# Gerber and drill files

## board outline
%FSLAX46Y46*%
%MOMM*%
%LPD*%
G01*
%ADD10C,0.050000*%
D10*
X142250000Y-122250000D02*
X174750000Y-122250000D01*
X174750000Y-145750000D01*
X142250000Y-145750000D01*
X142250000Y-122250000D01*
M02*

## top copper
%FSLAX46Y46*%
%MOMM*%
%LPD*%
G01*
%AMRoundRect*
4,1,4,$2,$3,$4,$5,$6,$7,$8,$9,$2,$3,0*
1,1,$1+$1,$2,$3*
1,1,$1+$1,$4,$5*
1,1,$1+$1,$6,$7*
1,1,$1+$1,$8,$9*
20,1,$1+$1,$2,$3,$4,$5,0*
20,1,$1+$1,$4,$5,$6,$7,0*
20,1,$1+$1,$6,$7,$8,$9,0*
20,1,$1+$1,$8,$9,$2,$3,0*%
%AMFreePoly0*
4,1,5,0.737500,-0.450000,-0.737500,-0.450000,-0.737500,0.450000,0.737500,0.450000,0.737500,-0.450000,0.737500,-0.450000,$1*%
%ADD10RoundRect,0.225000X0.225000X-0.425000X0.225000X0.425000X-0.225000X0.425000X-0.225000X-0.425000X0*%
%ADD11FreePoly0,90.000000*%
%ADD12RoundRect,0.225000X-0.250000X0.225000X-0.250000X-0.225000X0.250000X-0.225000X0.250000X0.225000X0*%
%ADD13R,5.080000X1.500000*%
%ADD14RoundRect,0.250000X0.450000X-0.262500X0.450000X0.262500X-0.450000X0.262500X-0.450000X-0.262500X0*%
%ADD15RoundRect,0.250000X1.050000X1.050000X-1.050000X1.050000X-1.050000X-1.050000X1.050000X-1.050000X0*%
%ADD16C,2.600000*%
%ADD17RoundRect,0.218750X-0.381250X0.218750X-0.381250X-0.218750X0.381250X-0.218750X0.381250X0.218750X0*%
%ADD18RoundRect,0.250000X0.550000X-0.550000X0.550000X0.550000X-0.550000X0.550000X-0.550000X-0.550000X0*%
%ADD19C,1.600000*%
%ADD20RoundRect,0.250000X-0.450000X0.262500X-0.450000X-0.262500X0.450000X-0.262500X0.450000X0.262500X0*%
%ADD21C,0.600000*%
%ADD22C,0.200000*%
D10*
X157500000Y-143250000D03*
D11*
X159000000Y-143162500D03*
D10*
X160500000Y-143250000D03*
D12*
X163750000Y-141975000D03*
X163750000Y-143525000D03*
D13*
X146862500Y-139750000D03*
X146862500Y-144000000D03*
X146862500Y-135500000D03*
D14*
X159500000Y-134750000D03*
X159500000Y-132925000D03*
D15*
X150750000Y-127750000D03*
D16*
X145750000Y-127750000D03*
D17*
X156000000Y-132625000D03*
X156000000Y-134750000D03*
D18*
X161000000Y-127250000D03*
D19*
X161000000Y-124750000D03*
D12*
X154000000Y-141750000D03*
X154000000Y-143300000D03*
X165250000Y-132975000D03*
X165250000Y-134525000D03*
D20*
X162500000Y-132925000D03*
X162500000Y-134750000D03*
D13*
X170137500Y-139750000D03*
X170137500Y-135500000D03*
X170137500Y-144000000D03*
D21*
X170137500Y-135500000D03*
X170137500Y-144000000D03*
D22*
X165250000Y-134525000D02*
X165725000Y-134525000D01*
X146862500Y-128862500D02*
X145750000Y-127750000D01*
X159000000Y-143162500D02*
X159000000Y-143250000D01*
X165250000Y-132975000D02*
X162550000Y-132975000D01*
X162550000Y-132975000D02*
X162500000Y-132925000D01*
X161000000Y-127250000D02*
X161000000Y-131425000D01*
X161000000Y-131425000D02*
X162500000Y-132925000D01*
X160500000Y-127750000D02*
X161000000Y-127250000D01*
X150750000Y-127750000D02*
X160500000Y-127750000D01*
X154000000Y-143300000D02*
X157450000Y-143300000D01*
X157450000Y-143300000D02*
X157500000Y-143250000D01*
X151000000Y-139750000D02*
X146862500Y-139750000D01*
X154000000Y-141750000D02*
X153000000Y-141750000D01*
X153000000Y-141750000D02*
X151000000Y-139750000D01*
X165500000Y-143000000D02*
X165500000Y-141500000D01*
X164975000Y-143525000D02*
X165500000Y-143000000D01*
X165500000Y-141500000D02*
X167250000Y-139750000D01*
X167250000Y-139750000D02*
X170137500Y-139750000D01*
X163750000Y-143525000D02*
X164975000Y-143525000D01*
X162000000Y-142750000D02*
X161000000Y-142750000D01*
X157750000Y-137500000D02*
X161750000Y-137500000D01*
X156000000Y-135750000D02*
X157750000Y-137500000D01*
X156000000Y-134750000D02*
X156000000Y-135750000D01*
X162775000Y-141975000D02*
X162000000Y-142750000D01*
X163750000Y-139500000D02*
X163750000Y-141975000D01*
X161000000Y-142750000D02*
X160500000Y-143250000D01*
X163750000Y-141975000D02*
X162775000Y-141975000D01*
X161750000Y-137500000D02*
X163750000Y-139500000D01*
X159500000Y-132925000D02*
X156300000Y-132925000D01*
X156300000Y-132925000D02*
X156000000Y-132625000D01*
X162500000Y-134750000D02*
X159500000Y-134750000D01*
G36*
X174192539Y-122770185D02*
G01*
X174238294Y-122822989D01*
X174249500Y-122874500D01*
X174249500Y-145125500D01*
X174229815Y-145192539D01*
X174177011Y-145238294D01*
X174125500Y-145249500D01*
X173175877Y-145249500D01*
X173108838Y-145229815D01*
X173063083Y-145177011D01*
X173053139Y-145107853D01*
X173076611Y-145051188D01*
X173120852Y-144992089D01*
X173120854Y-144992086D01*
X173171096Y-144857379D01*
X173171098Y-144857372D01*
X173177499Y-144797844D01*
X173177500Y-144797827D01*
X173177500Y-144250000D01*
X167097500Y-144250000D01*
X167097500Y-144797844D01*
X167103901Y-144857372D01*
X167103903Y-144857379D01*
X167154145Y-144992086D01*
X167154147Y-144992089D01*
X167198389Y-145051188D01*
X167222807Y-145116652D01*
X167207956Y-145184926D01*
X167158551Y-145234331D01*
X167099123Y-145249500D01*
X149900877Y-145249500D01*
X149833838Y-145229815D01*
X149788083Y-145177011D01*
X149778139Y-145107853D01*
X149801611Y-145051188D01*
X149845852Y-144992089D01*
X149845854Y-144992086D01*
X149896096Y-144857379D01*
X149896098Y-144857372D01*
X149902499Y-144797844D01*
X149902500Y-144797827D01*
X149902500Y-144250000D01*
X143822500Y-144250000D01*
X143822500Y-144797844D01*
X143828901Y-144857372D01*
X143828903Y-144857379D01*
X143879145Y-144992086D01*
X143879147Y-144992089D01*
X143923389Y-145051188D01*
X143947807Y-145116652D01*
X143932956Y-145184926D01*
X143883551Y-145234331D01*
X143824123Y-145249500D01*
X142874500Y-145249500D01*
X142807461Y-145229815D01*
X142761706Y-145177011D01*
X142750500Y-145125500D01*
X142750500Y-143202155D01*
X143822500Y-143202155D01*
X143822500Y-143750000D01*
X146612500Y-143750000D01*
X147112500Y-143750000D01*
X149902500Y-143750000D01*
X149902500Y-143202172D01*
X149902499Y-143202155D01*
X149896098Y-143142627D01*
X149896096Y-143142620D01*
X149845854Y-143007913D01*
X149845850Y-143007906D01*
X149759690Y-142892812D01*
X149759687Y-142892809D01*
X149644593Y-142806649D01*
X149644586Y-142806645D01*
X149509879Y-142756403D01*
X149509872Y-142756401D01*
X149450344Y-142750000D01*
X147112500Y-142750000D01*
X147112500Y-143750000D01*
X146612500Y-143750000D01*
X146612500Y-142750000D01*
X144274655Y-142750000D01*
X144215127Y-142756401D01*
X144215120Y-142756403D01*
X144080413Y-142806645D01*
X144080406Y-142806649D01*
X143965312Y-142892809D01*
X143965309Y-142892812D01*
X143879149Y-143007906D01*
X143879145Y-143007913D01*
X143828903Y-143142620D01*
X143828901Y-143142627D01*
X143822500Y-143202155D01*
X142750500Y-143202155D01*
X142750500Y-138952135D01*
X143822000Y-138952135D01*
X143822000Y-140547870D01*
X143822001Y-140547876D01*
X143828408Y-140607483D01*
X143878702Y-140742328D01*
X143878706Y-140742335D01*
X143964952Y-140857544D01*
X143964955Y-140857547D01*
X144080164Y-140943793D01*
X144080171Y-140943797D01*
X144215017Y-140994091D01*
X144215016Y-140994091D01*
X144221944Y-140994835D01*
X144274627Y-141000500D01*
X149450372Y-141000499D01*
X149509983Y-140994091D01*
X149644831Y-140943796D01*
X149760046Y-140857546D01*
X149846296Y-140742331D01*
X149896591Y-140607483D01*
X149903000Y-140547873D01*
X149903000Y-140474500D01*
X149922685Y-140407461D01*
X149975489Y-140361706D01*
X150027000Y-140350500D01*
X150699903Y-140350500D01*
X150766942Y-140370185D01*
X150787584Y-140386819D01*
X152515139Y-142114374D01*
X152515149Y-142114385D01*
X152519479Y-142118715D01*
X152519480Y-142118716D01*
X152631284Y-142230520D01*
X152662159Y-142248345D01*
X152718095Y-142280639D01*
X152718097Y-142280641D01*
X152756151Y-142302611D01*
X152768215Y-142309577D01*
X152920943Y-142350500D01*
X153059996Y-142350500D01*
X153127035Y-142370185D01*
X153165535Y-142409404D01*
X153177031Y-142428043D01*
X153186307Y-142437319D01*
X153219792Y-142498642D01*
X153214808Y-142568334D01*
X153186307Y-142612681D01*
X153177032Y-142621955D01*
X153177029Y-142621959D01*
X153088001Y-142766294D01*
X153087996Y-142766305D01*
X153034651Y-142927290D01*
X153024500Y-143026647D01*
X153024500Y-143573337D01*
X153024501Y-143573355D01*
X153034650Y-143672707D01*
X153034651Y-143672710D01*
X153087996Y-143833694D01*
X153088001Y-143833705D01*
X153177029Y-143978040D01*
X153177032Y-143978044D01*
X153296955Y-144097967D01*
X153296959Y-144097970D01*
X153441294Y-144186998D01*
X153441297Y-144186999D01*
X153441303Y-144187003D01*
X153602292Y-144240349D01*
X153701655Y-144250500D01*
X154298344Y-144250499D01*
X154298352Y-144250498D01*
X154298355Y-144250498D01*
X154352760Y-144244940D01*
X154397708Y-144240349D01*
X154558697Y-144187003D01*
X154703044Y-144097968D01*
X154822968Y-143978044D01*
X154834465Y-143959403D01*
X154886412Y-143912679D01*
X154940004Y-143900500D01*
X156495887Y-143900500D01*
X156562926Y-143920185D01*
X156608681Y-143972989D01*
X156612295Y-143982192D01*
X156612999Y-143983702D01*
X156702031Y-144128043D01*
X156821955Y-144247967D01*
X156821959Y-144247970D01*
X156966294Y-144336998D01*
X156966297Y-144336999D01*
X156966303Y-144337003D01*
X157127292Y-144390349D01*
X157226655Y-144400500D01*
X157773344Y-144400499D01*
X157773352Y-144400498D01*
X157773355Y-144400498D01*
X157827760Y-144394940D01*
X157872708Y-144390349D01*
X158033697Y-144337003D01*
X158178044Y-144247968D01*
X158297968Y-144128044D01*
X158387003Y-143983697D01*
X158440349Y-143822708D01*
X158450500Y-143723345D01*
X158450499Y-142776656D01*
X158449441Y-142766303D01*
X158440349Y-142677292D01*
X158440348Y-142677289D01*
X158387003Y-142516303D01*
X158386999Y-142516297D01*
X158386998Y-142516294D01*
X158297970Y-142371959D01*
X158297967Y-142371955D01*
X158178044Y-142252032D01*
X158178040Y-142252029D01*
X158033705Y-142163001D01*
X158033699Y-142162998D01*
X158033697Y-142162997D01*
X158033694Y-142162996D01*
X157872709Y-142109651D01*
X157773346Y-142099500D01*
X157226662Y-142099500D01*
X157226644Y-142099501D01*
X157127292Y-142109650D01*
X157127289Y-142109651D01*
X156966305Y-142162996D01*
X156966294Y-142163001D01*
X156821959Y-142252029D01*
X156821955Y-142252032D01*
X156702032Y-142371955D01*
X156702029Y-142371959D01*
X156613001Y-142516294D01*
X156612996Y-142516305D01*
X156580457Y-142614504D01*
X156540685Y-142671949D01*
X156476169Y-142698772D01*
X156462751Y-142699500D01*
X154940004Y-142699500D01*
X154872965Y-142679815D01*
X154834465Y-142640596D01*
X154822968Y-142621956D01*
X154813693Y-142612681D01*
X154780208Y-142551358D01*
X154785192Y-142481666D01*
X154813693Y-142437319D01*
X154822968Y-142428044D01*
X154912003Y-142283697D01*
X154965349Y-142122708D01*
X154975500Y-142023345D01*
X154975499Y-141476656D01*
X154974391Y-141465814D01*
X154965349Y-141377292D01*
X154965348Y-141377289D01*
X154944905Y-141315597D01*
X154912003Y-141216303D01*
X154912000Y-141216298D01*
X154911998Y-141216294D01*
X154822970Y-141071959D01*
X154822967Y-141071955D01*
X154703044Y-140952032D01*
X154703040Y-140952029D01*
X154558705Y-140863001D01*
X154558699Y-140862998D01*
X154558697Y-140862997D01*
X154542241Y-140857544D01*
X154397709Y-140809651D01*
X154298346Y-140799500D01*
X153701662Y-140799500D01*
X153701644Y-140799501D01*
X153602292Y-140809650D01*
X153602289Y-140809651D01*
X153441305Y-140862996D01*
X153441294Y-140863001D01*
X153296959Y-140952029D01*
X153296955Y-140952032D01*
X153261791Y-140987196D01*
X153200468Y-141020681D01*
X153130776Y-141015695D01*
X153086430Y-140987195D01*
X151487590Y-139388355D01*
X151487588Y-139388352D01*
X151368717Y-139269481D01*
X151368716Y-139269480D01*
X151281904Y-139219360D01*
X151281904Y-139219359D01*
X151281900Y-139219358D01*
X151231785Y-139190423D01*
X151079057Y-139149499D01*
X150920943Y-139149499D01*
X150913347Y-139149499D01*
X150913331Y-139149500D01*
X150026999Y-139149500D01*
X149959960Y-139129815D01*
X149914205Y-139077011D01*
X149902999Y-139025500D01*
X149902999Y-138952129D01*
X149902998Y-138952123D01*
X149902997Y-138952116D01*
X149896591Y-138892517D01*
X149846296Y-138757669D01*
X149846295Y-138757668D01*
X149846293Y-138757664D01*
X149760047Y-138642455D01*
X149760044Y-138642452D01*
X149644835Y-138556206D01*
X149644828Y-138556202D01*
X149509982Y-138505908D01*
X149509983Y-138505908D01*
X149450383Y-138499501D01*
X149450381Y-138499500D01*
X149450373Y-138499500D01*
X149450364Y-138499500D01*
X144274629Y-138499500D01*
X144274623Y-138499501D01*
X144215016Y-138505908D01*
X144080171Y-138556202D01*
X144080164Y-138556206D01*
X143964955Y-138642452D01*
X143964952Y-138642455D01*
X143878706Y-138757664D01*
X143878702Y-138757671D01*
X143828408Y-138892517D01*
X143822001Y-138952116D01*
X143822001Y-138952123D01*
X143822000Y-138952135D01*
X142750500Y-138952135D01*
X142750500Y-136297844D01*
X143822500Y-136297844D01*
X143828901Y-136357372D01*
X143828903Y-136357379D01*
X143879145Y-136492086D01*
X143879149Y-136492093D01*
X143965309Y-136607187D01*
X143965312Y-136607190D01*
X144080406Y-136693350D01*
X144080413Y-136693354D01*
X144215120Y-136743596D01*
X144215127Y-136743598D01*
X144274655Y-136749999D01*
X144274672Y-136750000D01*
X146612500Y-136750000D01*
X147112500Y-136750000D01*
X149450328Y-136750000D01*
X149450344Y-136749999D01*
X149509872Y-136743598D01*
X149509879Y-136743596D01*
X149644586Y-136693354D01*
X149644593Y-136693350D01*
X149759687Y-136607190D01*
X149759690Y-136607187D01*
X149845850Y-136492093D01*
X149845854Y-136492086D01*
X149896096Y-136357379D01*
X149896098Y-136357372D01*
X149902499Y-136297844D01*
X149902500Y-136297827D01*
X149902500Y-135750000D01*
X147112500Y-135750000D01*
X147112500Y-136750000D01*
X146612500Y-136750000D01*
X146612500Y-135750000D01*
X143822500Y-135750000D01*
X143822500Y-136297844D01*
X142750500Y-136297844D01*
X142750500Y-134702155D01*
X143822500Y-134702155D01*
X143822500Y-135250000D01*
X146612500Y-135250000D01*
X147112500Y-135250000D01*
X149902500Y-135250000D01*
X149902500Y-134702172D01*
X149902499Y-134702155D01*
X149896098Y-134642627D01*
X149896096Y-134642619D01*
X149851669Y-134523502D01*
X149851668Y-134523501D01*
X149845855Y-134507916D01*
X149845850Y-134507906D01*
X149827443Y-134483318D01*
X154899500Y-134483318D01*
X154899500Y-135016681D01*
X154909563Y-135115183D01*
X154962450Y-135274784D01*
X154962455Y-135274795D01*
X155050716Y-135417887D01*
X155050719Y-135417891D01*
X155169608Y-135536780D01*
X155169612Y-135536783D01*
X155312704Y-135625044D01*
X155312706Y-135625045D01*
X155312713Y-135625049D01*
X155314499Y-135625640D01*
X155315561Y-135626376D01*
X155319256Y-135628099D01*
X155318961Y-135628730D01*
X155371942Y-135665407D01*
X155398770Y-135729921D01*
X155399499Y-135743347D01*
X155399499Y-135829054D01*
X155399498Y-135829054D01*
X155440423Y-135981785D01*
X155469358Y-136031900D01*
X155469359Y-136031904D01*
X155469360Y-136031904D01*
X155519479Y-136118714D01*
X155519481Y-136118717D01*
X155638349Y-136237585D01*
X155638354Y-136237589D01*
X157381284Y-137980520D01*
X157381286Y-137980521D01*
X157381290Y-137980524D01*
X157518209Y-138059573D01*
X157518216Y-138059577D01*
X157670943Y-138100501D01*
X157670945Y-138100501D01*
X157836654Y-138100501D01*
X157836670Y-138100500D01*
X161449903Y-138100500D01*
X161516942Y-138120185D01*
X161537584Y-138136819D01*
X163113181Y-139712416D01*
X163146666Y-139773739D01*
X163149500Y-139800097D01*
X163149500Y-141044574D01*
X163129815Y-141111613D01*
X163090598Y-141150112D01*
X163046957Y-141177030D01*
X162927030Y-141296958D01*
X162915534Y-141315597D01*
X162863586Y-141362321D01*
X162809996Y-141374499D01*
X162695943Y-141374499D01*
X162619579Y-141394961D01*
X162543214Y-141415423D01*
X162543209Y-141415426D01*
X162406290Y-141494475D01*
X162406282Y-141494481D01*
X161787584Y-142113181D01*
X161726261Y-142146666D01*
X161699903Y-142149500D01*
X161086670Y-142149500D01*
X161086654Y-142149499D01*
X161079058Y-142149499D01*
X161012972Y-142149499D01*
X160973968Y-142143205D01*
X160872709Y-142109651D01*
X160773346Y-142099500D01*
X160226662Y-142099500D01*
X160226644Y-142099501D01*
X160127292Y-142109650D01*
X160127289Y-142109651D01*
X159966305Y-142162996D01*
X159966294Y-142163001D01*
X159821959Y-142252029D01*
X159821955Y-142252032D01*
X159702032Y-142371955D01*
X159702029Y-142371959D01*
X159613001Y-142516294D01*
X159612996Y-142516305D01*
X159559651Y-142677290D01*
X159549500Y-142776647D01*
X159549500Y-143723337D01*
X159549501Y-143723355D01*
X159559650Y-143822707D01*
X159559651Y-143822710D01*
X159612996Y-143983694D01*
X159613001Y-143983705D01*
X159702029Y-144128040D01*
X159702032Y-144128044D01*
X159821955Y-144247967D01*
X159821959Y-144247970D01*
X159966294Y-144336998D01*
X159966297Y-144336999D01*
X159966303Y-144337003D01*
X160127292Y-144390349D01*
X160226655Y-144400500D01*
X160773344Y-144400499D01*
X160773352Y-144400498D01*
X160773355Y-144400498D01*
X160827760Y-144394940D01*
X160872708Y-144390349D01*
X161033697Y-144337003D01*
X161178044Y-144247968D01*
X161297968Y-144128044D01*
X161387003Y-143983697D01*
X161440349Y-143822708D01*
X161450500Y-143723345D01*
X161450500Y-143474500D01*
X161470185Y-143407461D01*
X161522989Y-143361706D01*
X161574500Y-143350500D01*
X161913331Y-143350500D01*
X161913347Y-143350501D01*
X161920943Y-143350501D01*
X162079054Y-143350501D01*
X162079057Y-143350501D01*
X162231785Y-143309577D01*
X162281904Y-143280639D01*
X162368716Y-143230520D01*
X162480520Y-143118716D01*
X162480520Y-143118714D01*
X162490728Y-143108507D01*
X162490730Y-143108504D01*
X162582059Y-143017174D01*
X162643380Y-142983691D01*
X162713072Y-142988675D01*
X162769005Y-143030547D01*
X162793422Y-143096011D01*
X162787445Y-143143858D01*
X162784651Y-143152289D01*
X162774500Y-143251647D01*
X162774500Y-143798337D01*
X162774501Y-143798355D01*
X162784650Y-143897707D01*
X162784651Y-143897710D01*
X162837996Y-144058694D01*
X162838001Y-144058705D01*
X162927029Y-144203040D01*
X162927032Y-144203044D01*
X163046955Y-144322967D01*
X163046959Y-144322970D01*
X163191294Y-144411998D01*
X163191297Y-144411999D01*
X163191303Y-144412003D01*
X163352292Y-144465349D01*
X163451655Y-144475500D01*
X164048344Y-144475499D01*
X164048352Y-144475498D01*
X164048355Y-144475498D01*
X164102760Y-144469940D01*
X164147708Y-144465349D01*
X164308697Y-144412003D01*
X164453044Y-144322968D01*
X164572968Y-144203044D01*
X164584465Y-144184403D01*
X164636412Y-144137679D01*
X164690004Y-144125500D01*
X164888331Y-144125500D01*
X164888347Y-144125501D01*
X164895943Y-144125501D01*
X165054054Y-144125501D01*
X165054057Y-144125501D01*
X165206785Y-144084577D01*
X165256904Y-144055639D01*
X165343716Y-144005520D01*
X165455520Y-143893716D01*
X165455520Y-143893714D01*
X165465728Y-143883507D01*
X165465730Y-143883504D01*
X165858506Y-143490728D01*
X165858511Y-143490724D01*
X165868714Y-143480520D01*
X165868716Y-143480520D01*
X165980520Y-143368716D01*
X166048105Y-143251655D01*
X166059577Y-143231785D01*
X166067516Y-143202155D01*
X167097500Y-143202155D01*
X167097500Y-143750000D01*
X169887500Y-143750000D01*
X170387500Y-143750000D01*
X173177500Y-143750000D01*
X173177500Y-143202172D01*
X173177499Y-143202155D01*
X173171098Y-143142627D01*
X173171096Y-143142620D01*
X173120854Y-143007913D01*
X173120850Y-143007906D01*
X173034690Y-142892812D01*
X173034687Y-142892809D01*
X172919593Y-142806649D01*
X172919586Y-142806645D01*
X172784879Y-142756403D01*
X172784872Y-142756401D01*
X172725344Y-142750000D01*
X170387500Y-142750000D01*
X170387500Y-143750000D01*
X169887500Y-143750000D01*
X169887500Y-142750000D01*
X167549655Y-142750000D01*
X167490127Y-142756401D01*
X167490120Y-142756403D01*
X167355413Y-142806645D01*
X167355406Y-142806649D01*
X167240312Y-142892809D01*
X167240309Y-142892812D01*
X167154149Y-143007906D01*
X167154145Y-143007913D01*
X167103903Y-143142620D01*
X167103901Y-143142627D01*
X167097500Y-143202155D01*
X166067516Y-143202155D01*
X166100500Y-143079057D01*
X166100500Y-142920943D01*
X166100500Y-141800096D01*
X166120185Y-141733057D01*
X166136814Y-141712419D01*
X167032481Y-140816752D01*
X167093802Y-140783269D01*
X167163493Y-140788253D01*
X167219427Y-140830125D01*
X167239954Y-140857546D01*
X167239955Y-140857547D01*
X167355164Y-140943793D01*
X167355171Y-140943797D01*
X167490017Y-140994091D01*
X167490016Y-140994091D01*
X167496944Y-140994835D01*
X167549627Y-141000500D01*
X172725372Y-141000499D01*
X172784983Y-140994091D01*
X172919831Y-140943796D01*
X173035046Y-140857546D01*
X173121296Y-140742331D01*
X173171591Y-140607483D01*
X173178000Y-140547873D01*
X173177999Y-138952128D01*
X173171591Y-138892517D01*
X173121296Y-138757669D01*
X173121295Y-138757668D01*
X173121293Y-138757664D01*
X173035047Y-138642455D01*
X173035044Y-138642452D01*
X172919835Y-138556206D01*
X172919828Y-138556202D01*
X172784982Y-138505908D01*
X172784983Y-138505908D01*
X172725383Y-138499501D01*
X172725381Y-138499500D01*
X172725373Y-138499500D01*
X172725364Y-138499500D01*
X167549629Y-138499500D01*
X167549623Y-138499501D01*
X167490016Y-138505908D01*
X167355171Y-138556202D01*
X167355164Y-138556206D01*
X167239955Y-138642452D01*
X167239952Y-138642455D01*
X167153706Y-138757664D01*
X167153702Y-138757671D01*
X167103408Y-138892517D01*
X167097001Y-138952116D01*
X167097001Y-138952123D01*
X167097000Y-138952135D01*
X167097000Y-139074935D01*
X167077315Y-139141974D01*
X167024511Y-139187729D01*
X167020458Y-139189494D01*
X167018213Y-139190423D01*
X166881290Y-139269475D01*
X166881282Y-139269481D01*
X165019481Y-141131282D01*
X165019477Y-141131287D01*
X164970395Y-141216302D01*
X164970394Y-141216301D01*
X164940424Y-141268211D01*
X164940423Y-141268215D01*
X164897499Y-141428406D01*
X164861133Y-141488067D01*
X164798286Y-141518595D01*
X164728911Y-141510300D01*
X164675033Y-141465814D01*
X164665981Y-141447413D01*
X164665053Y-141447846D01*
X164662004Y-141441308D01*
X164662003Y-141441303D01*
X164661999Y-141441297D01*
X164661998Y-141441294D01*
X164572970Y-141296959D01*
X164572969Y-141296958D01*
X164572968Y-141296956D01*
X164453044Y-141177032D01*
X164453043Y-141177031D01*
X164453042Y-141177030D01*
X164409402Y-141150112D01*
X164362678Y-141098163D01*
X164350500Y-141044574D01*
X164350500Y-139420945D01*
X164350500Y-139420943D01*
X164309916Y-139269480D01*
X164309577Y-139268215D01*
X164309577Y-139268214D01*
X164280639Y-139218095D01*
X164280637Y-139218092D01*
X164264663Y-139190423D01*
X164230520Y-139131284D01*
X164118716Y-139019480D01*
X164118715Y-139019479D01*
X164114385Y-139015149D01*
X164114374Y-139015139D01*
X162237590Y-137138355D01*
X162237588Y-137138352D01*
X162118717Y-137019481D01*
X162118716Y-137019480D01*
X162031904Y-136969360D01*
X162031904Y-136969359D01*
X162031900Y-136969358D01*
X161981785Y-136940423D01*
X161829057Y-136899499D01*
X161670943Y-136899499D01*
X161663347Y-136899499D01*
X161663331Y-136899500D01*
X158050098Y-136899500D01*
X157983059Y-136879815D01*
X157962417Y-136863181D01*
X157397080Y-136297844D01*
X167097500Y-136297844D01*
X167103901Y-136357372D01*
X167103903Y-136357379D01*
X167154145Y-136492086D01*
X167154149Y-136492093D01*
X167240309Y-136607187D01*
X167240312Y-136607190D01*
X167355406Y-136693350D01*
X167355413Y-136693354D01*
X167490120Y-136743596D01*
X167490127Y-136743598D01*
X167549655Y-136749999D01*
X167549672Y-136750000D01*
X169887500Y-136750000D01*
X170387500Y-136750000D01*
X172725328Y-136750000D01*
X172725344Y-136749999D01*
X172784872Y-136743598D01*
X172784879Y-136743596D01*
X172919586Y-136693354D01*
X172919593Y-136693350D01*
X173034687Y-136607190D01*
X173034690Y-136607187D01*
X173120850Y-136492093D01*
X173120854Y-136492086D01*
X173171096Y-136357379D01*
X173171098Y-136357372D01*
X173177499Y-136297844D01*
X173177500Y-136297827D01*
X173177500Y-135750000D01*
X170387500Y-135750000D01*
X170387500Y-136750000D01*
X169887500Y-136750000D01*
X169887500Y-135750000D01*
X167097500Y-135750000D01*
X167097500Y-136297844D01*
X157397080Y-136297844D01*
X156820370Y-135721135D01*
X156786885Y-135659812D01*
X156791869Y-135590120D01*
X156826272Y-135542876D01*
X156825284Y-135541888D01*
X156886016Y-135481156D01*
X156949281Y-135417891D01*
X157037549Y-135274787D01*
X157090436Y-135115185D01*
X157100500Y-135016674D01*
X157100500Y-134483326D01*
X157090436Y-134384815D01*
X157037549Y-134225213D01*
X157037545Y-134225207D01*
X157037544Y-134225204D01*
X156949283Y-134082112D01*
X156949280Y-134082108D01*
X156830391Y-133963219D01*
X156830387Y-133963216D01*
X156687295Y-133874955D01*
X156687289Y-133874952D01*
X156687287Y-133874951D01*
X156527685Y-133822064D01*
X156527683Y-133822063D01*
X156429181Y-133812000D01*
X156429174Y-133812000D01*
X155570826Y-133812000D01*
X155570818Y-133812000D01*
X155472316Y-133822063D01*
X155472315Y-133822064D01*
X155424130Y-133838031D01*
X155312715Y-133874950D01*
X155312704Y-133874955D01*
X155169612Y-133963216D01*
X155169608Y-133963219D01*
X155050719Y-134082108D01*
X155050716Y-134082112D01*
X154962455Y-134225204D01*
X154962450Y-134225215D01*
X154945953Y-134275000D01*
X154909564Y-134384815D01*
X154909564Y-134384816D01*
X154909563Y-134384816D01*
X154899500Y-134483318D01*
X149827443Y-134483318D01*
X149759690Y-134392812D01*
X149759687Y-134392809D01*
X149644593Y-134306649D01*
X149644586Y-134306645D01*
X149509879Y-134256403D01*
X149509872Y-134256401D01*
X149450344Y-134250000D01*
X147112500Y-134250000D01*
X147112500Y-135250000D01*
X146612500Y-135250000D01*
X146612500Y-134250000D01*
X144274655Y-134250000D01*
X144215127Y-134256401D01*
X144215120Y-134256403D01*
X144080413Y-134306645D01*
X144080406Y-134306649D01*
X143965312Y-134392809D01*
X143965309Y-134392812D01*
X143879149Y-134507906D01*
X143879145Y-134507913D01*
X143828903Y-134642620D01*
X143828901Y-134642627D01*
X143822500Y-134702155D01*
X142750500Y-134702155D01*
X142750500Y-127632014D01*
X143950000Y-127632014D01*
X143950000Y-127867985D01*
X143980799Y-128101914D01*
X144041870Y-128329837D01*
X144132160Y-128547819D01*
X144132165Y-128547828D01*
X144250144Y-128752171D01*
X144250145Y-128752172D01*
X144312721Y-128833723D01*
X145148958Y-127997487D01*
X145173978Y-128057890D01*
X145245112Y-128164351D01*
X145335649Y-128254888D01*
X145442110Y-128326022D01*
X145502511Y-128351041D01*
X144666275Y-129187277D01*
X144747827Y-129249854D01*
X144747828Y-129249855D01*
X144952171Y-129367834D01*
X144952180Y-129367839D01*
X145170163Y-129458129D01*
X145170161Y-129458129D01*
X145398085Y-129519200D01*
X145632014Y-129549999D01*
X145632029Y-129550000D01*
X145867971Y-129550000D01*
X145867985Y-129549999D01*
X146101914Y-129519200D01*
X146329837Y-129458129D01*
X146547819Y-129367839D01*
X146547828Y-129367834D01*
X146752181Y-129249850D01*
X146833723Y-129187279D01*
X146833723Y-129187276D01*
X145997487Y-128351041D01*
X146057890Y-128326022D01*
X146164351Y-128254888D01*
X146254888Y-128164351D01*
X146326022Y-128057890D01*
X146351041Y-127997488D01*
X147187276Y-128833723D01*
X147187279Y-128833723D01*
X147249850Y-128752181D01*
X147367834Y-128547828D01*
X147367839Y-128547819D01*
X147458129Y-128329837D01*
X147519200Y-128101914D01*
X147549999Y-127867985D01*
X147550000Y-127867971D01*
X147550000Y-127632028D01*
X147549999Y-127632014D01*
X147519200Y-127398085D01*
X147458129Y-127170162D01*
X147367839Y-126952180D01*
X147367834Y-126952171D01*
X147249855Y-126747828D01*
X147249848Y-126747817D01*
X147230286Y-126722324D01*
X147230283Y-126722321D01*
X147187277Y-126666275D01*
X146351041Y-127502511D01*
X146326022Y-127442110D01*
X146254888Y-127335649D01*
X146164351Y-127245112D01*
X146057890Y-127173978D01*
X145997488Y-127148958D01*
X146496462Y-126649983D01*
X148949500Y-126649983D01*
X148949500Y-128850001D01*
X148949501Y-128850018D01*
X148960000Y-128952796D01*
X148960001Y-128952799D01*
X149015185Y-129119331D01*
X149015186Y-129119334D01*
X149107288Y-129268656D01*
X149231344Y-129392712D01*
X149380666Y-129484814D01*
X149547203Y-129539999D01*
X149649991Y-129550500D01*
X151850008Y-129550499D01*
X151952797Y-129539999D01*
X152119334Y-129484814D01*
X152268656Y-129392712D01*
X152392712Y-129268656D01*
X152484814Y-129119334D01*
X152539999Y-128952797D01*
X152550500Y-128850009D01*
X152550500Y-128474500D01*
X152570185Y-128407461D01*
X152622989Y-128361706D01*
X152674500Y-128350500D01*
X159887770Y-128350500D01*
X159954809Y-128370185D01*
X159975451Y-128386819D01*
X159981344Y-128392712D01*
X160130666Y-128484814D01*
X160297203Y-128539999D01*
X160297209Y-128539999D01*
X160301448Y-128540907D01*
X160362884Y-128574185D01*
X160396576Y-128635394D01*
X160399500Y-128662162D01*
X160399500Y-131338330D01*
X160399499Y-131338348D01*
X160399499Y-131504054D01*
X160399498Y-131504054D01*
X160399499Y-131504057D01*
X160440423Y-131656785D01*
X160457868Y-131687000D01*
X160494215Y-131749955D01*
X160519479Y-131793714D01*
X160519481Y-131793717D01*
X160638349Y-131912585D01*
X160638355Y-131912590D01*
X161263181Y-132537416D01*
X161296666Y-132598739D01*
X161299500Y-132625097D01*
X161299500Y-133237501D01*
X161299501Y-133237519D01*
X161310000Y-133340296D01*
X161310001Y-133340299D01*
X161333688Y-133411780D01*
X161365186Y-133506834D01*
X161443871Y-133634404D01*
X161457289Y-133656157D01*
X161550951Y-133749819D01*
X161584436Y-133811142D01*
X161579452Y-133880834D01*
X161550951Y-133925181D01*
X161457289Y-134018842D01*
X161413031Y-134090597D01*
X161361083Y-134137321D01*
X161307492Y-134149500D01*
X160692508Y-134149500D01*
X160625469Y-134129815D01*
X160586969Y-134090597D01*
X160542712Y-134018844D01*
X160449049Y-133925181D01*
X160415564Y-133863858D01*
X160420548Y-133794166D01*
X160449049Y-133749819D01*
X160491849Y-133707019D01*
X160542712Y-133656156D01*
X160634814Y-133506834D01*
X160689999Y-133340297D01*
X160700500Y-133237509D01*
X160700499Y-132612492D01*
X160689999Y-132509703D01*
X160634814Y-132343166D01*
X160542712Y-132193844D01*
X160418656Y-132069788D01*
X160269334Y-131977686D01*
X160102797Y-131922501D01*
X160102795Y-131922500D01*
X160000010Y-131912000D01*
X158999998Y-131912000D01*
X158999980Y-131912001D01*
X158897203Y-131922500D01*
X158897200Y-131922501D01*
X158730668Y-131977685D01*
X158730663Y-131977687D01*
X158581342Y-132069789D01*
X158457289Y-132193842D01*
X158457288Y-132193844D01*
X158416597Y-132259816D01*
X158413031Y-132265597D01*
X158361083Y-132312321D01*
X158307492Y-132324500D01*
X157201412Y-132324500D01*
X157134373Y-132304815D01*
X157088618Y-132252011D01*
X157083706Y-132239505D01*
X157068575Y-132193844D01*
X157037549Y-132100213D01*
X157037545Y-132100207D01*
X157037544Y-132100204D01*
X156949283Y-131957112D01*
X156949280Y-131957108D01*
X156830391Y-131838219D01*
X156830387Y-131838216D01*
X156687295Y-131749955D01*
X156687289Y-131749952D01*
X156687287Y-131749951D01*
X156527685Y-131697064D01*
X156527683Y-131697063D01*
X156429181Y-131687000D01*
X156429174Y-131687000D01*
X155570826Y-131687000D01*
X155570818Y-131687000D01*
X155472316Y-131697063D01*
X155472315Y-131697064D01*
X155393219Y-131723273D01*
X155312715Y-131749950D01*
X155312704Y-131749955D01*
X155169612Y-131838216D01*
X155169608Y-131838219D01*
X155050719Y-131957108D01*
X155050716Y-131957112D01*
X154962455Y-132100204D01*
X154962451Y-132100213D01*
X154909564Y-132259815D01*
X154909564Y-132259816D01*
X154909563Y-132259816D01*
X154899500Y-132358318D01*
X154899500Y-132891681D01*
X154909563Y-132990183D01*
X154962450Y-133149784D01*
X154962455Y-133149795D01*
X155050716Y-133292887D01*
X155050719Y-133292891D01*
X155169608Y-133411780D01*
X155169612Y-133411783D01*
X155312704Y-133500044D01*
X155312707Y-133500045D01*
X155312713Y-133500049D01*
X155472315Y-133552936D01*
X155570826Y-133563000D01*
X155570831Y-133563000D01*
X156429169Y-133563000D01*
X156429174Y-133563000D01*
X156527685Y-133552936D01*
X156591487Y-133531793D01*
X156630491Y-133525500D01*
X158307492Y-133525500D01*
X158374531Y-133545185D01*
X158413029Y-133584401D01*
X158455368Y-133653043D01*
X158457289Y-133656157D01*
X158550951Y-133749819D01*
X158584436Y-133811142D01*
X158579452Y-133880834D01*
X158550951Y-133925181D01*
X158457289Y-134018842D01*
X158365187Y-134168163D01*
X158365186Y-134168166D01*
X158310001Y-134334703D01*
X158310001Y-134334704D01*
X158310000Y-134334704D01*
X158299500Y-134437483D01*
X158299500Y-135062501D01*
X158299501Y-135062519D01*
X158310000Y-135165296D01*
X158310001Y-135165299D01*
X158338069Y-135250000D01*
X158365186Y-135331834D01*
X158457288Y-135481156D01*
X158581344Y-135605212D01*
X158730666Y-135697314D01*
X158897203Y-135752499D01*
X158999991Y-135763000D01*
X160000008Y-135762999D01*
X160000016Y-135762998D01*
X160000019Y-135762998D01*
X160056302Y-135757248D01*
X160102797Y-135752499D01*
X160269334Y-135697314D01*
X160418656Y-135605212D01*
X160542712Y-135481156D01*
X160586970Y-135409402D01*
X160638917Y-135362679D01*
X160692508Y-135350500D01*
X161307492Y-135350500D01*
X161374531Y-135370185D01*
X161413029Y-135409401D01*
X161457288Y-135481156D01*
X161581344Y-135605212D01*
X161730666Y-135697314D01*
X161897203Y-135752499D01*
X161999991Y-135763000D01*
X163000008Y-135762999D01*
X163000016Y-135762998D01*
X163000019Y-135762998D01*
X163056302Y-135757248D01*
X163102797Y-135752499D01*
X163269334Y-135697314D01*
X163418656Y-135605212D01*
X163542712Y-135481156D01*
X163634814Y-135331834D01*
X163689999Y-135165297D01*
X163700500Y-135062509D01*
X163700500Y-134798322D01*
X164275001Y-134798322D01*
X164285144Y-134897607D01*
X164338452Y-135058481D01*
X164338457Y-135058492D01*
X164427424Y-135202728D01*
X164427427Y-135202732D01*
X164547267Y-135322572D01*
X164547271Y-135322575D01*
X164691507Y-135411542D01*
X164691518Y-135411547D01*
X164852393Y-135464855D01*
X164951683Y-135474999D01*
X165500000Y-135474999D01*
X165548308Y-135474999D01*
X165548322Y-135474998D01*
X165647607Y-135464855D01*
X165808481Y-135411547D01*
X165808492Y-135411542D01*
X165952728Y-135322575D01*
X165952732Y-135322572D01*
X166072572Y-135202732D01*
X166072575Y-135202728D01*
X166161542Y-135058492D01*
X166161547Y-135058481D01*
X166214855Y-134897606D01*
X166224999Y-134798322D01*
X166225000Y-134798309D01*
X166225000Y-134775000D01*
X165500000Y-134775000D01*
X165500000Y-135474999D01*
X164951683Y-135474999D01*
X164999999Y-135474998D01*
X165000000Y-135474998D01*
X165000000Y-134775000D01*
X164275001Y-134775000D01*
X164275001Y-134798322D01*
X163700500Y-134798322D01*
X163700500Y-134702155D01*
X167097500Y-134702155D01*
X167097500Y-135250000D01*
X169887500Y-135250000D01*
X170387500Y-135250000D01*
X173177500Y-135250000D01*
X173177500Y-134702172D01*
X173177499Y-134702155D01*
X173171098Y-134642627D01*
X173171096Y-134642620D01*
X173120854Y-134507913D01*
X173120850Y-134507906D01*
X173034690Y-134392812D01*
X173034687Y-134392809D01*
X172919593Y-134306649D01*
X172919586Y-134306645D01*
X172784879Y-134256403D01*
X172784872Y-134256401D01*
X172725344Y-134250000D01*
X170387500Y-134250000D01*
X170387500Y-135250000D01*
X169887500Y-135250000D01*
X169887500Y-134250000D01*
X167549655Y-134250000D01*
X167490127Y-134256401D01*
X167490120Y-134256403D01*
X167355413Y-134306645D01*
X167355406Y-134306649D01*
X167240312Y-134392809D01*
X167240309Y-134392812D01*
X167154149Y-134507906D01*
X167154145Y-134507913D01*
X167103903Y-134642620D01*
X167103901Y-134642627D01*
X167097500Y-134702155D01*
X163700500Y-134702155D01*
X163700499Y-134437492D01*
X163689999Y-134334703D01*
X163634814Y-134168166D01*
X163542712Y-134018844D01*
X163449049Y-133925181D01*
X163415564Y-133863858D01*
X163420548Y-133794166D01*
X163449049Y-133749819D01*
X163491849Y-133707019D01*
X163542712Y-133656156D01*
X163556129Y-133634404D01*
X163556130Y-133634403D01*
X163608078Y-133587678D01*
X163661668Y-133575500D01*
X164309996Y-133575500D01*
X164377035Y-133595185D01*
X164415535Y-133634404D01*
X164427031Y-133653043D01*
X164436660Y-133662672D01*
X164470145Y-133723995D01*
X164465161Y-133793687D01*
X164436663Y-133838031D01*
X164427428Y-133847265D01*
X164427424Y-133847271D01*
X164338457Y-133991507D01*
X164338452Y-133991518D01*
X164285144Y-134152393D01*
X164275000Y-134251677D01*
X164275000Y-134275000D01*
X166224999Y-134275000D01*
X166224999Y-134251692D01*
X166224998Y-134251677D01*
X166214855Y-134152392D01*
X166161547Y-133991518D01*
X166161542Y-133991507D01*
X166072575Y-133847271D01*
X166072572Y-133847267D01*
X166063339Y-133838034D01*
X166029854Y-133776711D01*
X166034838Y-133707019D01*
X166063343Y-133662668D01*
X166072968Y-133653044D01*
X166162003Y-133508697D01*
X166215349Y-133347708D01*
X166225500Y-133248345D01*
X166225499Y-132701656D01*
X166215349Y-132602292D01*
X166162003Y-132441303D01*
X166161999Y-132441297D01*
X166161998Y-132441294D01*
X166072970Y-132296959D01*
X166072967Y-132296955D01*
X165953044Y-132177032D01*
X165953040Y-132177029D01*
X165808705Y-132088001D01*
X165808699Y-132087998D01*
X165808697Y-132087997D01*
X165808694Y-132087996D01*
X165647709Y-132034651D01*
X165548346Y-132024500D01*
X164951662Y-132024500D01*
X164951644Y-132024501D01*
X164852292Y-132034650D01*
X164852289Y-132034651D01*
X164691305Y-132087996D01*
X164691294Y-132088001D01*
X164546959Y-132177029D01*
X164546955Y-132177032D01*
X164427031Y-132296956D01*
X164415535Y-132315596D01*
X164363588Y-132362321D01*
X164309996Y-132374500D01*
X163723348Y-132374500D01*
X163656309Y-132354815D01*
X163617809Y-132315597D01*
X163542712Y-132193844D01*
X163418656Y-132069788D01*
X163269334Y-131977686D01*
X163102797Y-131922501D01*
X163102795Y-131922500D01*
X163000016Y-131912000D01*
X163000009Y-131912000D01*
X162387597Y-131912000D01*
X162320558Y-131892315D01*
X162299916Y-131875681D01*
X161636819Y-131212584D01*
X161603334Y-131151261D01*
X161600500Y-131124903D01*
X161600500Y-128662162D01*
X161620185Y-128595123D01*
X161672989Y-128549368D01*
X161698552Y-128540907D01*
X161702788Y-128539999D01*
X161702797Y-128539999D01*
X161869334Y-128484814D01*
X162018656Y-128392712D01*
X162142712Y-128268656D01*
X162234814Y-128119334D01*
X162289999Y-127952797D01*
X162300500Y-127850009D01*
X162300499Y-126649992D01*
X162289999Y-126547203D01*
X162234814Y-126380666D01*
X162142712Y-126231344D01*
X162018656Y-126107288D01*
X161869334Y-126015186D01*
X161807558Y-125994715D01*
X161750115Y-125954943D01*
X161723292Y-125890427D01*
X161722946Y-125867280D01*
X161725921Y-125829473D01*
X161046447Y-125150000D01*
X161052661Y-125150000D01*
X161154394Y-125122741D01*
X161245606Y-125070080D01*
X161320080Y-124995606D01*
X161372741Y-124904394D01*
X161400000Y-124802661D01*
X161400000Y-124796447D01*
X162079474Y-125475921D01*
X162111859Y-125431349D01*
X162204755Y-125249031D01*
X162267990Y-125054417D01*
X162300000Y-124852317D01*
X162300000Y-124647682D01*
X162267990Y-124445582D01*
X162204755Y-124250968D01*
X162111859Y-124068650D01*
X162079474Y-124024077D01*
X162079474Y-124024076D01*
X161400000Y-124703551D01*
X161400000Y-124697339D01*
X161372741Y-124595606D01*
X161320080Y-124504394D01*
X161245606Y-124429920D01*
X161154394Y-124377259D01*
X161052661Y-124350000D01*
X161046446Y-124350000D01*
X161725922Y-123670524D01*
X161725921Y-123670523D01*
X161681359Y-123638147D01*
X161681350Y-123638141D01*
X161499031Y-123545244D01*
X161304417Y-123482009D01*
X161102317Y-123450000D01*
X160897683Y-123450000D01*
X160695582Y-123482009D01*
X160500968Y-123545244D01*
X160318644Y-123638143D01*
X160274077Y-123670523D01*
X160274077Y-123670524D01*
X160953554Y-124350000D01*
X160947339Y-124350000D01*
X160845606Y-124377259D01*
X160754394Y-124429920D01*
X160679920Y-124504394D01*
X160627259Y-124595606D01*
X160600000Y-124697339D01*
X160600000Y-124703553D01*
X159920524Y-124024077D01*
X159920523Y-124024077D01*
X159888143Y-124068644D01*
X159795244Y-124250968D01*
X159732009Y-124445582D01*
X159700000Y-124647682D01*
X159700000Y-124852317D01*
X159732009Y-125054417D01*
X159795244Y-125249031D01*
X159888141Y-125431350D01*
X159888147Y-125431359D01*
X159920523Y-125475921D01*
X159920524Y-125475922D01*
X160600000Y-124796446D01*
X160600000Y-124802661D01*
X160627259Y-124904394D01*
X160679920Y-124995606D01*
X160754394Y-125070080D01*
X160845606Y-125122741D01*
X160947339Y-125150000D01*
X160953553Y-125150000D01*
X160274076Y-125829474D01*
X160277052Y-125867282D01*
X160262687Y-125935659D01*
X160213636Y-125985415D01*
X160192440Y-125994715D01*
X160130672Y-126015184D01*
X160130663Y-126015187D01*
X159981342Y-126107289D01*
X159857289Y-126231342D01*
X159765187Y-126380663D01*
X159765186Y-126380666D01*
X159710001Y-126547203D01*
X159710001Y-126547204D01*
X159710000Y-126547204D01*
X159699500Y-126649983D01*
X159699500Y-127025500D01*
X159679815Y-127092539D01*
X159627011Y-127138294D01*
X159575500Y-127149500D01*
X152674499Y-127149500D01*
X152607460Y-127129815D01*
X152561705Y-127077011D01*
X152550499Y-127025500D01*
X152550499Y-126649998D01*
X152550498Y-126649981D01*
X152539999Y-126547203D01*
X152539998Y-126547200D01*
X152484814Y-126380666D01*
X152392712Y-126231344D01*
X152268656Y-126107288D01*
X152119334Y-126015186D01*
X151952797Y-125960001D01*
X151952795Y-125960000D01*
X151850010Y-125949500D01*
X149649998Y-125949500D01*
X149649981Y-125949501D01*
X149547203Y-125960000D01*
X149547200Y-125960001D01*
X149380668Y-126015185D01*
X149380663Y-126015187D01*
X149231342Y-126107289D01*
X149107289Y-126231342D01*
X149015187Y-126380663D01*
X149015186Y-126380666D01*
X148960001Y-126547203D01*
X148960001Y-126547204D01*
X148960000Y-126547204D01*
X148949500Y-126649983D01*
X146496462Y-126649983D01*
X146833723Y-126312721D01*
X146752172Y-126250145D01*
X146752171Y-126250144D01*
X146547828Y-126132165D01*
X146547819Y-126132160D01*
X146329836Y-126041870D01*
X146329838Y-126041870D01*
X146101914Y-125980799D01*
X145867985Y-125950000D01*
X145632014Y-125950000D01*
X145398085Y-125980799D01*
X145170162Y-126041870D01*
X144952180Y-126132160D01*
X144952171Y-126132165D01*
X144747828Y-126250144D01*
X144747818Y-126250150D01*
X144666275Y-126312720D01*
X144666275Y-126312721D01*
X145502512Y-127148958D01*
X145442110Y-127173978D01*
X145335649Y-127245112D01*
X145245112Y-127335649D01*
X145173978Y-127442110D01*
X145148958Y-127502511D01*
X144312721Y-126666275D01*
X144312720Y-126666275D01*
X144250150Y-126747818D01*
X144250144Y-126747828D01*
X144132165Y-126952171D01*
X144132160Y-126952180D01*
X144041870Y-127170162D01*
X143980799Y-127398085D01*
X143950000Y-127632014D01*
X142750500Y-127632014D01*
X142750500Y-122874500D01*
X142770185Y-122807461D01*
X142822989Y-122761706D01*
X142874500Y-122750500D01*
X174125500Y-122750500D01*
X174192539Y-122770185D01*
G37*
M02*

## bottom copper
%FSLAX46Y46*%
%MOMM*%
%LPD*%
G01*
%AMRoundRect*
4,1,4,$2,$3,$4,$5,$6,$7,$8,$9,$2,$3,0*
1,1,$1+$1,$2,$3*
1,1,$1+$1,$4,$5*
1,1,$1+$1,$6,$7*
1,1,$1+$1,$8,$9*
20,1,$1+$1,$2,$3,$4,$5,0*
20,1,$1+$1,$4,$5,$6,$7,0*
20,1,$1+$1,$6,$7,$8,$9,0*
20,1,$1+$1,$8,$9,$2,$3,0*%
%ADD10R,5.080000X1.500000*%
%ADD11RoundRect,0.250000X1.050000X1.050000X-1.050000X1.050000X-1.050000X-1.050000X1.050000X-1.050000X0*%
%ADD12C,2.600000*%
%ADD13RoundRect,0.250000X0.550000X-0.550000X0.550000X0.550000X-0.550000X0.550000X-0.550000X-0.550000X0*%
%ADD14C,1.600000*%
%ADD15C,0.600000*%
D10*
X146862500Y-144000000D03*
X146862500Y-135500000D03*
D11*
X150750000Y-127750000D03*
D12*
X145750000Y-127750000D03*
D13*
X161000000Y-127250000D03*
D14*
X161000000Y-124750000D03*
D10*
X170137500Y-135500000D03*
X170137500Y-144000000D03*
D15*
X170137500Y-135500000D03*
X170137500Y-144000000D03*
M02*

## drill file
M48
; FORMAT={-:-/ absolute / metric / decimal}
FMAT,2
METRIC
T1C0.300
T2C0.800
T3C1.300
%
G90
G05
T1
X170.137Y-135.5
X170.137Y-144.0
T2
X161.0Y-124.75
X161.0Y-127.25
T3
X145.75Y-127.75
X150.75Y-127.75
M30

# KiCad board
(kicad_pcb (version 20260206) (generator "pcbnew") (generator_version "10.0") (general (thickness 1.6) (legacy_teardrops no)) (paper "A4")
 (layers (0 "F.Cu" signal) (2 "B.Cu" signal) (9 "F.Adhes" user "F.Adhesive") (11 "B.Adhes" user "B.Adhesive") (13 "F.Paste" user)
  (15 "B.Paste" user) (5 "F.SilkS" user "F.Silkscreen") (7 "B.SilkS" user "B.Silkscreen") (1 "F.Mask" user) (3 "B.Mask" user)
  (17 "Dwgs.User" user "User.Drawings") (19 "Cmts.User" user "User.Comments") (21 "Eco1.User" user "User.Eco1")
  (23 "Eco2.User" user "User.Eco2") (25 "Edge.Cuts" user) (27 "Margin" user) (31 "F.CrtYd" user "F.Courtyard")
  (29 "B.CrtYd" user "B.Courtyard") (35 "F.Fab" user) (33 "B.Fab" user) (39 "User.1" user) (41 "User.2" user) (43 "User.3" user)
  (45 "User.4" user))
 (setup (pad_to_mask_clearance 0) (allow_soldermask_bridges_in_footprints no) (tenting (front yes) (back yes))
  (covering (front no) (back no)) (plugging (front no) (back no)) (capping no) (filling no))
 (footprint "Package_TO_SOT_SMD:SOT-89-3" (layer "F.Cu") (at 159 141.3 90)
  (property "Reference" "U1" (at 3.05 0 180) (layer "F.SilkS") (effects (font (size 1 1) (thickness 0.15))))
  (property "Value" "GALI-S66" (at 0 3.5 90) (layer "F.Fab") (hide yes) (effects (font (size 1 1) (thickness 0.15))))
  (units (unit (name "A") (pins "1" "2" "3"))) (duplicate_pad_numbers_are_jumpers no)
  (pad "1" smd roundrect (at -1.95 -1.5 90) (size 1.3 0.9) (layers "F.Cu" "F.Mask" "F.Paste") (roundrect_rratio 0.25) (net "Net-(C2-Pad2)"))
  (pad "2" smd custom (at -1.8625 0 90) (size 1.475 0.9) (layers "F.Cu" "F.Mask" "F.Paste") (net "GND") (zone_connect 2)
   (thermal_bridge_angle 45) (options (clearance outline) (anchor rect)) (primitives))
  (pad "3" smd roundrect (at -1.95 1.5 90) (size 1.3 0.9) (layers "F.Cu" "F.Mask" "F.Paste") (roundrect_rratio 0.25) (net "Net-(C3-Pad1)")))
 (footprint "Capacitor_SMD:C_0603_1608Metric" (layer "F.Cu") (at 163.75 142.75 -90)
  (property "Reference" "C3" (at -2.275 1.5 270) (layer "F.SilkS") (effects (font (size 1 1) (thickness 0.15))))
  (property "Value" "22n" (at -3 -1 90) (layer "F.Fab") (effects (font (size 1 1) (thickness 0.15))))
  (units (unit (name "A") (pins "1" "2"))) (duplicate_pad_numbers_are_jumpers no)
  (pad "1" smd roundrect (at -0.775 0 270) (size 0.9 0.95) (layers "F.Cu" "F.Mask" "F.Paste") (roundrect_rratio 0.25) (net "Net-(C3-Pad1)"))
  (pad "2" smd roundrect (at 0.775 0 270) (size 0.9 0.95) (layers "F.Cu" "F.Mask" "F.Paste") (roundrect_rratio 0.25) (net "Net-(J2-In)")))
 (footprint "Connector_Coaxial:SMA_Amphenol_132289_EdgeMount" (layer "F.Cu") (at 146.8625 139.75 180)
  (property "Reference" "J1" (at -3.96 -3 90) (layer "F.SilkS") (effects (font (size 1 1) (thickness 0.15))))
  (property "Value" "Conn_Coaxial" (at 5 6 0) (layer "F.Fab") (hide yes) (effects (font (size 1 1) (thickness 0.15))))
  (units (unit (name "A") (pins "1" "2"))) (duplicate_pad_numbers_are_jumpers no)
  (pad "1" smd rect (at 0 0 270) (size 1.5 5.08) (layers "F.Cu" "F.Mask" "F.Paste") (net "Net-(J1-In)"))
  (pad "2" smd rect (at 0 -4.25 270) (size 1.5 5.08) (layers "F.Cu" "F.Mask" "F.Paste") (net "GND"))
  (pad "2" smd rect (at 0 -4.25 270) (size 1.5 5.08) (layers "B.Cu" "B.Mask" "B.Paste") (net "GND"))
  (pad "2" smd rect (at 0 4.25 270) (size 1.5 5.08) (layers "F.Cu" "F.Mask" "F.Paste") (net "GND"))
  (pad "2" smd rect (at 0 4.25 270) (size 1.5 5.08) (layers "B.Cu" "B.Mask" "B.Paste") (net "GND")))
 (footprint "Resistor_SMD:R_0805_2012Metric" (layer "F.Cu") (at 159.5 133.8375 90)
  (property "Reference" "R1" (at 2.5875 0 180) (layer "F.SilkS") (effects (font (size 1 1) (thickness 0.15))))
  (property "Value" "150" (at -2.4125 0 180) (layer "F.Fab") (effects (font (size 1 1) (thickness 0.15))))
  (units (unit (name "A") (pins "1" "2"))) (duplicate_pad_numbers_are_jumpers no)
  (pad "1" smd roundrect (at -0.9125 0 90) (size 1.025 1.4) (layers "F.Cu" "F.Mask" "F.Paste") (roundrect_rratio 0.243902)
   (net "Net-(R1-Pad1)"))
  (pad "2" smd roundrect (at 0.9125 0 90) (size 1.025 1.4) (layers "F.Cu" "F.Mask" "F.Paste") (roundrect_rratio 0.243902)
   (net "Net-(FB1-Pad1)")))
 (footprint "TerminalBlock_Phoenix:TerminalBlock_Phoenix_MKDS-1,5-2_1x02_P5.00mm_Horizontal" (layer "F.Cu") (at 150.75 127.75 180)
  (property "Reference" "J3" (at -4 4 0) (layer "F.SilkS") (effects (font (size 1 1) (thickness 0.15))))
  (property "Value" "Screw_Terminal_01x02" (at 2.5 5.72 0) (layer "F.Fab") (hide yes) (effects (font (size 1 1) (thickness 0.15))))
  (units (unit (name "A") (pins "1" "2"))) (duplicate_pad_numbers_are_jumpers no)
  (pad "1" thru_hole roundrect (at 0 0 180) (size 2.6 2.6) (drill 1.3) (layers "*.Cu" "*.Mask") (remove_unused_layers no)
   (roundrect_rratio 0.096154) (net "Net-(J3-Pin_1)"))
  (pad "2" thru_hole circle (at 5 0 180) (size 2.6 2.6) (drill 1.3) (layers "*.Cu" "*.Mask") (remove_unused_layers no) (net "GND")))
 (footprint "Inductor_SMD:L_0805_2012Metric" (layer "F.Cu") (at 156 133.6875 -90)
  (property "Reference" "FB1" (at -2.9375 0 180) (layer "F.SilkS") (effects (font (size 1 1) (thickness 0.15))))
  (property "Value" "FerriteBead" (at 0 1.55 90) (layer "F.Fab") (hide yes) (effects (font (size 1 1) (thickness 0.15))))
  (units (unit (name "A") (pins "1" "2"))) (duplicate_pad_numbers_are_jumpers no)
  (pad "1" smd roundrect (at -1.0625 0 270) (size 0.875 1.2) (layers "F.Cu" "F.Mask" "F.Paste") (roundrect_rratio 0.25)
   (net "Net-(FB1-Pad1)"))
  (pad "2" smd roundrect (at 1.0625 0 270) (size 0.875 1.2) (layers "F.Cu" "F.Mask" "F.Paste") (roundrect_rratio 0.25) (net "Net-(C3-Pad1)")))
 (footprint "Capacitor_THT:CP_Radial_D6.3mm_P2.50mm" (layer "F.Cu") (at 161 127.25 90)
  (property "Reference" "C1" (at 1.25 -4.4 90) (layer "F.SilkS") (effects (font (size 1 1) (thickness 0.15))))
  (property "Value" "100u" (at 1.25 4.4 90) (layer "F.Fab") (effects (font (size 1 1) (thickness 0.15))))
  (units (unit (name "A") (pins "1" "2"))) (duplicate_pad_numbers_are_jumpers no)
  (pad "1" thru_hole roundrect (at 0 0 90) (size 1.6 1.6) (drill 0.8) (layers "*.Cu" "*.Mask") (remove_unused_layers no)
   (roundrect_rratio 0.15625) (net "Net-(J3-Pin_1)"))
  (pad "2" thru_hole circle (at 2.5 0 90) (size 1.6 1.6) (drill 0.8) (layers "*.Cu" "*.Mask") (remove_unused_layers no) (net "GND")))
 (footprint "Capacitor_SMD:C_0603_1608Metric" (layer "F.Cu") (at 154 142.525 -90)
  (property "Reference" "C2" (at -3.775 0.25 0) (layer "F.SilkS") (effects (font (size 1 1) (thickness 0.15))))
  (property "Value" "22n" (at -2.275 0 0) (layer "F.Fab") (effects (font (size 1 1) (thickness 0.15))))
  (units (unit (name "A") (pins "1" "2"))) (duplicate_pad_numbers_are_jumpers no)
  (pad "1" smd roundrect (at -0.775 0 270) (size 0.9 0.95) (layers "F.Cu" "F.Mask" "F.Paste") (roundrect_rratio 0.25) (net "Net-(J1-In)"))
  (pad "2" smd roundrect (at 0.775 0 270) (size 0.9 0.95) (layers "F.Cu" "F.Mask" "F.Paste") (roundrect_rratio 0.25) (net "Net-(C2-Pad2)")))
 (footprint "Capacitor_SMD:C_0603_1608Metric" (layer "F.Cu") (at 165.25 133.75 -90)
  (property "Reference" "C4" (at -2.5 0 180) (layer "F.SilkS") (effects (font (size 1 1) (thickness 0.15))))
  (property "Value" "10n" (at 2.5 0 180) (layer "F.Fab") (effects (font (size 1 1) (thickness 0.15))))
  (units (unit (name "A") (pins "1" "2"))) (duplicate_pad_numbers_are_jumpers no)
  (pad "1" smd roundrect (at -0.775 0 270) (size 0.9 0.95) (layers "F.Cu" "F.Mask" "F.Paste") (roundrect_rratio 0.25) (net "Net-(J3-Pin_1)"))
  (pad "2" smd roundrect (at 0.775 0 270) (size 0.9 0.95) (layers "F.Cu" "F.Mask" "F.Paste") (roundrect_rratio 0.25) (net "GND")))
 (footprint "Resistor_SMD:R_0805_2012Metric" (layer "F.Cu") (at 162.5 133.8375 -90)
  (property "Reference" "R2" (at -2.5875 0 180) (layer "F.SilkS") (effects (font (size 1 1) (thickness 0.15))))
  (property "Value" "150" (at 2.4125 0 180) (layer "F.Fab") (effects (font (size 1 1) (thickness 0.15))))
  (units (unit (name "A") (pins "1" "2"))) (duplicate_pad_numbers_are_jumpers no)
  (pad "1" smd roundrect (at -0.9125 0 270) (size 1.025 1.4) (layers "F.Cu" "F.Mask" "F.Paste") (roundrect_rratio 0.243902)
   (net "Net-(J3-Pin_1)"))
  (pad "2" smd roundrect (at 0.9125 0 270) (size 1.025 1.4) (layers "F.Cu" "F.Mask" "F.Paste") (roundrect_rratio 0.243902)
   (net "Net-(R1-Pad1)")))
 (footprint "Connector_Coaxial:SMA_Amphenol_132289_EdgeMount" (layer "F.Cu") (at 170.1375 139.75)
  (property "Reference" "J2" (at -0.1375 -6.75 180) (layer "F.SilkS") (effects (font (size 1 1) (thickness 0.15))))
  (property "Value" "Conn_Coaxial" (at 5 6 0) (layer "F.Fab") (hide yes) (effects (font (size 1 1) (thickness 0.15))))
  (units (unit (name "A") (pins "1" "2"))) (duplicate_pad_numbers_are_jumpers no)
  (pad "1" smd rect (at 0 0 90) (size 1.5 5.08) (layers "F.Cu" "F.Mask" "F.Paste") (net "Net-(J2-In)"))
  (pad "2" smd rect (at 0 -4.25 90) (size 1.5 5.08) (layers "F.Cu" "F.Mask" "F.Paste") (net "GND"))
  (pad "2" smd rect (at 0 -4.25 90) (size 1.5 5.08) (layers "B.Cu" "B.Mask" "B.Paste") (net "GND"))
  (pad "2" smd rect (at 0 4.25 90) (size 1.5 5.08) (layers "F.Cu" "F.Mask" "F.Paste") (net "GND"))
  (pad "2" smd rect (at 0 4.25 90) (size 1.5 5.08) (layers "B.Cu" "B.Mask" "B.Paste") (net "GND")))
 (gr_rect (start 142.25 122.25) (end 174.75 145.75) (stroke (width 0.05) (type default)) (fill no) (layer "Edge.Cuts"))
 (segment (start 165.25 134.525) (end 165.725 134.525) (width 0.2) (layer "F.Cu") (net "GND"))
 (segment (start 146.8625 128.8625) (end 145.75 127.75) (width 0.2) (layer "F.Cu") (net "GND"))
 (segment (start 159 143.1625) (end 159 143.25) (width 0.2) (layer "F.Cu") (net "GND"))
 (via (at 170.1375 135.5) (size 0.6) (drill 0.3) (layers "F.Cu" "B.Cu") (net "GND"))
 (via (at 170.1375 144) (size 0.6) (drill 0.3) (layers "F.Cu" "B.Cu") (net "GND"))
 (segment (start 165.25 132.975) (end 162.55 132.975) (width 0.2) (layer "F.Cu") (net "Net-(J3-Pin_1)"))
 (segment (start 162.55 132.975) (end 162.5 132.925) (width 0.2) (layer "F.Cu") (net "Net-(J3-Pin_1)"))
 (segment (start 161 127.25) (end 161 131.425) (width 0.2) (layer "F.Cu") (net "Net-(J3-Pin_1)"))
 (segment (start 161 131.425) (end 162.5 132.925) (width 0.2) (layer "F.Cu") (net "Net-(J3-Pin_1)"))
 (segment (start 160.5 127.75) (end 161 127.25) (width 0.2) (layer "F.Cu") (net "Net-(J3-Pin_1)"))
 (segment (start 150.75 127.75) (end 160.5 127.75) (width 0.2) (layer "F.Cu") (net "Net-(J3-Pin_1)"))
 (segment (start 154 143.3) (end 157.45 143.3) (width 0.2) (layer "F.Cu") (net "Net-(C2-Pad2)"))
 (segment (start 157.45 143.3) (end 157.5 143.25) (width 0.2) (layer "F.Cu") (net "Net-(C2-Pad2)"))
 (segment (start 151 139.75) (end 146.8625 139.75) (width 0.2) (layer "F.Cu") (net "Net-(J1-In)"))
 (segment (start 154 141.75) (end 153 141.75) (width 0.2) (layer "F.Cu") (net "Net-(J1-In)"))
 (segment (start 153 141.75) (end 151 139.75) (width 0.2) (layer "F.Cu") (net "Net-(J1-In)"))
 (segment (start 165.5 143) (end 165.5 141.5) (width 0.2) (layer "F.Cu") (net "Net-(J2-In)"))
 (segment (start 164.975 143.525) (end 165.5 143) (width 0.2) (layer "F.Cu") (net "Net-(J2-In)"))
 (segment (start 165.5 141.5) (end 167.25 139.75) (width 0.2) (layer "F.Cu") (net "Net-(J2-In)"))
 (segment (start 167.25 139.75) (end 170.1375 139.75) (width 0.2) (layer "F.Cu") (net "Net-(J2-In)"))
 (segment (start 163.75 143.525) (end 164.975 143.525) (width 0.2) (layer "F.Cu") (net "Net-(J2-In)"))
 (segment (start 162 142.75) (end 161 142.75) (width 0.2) (layer "F.Cu") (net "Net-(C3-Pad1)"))
 (segment (start 157.75 137.5) (end 161.75 137.5) (width 0.2) (layer "F.Cu") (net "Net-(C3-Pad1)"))
 (segment (start 156 135.75) (end 157.75 137.5) (width 0.2) (layer "F.Cu") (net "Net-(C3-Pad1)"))
 (segment (start 156 134.75) (end 156 135.75) (width 0.2) (layer "F.Cu") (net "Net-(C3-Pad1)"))
 (segment (start 162.775 141.975) (end 162 142.75) (width 0.2) (layer "F.Cu") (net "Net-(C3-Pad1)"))
 (segment (start 163.75 139.5) (end 163.75 141.975) (width 0.2) (layer "F.Cu") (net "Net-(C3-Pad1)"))
 (segment (start 161 142.75) (end 160.5 143.25) (width 0.2) (layer "F.Cu") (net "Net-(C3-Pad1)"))
 (segment (start 163.75 141.975) (end 162.775 141.975) (width 0.2) (layer "F.Cu") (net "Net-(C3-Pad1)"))
 (segment (start 161.75 137.5) (end 163.75 139.5) (width 0.2) (layer "F.Cu") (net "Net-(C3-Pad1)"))
 (segment (start 159.5 132.925) (end 156.3 132.925) (width 0.2) (layer "F.Cu") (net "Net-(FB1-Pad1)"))
 (segment (start 156.3 132.925) (end 156 132.625) (width 0.2) (layer "F.Cu") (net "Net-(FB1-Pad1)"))
 (segment (start 162.5 134.75) (end 159.5 134.75) (width 0.2) (layer "F.Cu") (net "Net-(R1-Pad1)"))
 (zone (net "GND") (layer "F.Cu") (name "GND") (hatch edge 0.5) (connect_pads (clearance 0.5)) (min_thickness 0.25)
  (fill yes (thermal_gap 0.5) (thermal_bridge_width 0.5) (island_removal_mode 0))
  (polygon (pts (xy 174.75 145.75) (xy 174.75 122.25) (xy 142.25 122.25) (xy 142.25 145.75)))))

